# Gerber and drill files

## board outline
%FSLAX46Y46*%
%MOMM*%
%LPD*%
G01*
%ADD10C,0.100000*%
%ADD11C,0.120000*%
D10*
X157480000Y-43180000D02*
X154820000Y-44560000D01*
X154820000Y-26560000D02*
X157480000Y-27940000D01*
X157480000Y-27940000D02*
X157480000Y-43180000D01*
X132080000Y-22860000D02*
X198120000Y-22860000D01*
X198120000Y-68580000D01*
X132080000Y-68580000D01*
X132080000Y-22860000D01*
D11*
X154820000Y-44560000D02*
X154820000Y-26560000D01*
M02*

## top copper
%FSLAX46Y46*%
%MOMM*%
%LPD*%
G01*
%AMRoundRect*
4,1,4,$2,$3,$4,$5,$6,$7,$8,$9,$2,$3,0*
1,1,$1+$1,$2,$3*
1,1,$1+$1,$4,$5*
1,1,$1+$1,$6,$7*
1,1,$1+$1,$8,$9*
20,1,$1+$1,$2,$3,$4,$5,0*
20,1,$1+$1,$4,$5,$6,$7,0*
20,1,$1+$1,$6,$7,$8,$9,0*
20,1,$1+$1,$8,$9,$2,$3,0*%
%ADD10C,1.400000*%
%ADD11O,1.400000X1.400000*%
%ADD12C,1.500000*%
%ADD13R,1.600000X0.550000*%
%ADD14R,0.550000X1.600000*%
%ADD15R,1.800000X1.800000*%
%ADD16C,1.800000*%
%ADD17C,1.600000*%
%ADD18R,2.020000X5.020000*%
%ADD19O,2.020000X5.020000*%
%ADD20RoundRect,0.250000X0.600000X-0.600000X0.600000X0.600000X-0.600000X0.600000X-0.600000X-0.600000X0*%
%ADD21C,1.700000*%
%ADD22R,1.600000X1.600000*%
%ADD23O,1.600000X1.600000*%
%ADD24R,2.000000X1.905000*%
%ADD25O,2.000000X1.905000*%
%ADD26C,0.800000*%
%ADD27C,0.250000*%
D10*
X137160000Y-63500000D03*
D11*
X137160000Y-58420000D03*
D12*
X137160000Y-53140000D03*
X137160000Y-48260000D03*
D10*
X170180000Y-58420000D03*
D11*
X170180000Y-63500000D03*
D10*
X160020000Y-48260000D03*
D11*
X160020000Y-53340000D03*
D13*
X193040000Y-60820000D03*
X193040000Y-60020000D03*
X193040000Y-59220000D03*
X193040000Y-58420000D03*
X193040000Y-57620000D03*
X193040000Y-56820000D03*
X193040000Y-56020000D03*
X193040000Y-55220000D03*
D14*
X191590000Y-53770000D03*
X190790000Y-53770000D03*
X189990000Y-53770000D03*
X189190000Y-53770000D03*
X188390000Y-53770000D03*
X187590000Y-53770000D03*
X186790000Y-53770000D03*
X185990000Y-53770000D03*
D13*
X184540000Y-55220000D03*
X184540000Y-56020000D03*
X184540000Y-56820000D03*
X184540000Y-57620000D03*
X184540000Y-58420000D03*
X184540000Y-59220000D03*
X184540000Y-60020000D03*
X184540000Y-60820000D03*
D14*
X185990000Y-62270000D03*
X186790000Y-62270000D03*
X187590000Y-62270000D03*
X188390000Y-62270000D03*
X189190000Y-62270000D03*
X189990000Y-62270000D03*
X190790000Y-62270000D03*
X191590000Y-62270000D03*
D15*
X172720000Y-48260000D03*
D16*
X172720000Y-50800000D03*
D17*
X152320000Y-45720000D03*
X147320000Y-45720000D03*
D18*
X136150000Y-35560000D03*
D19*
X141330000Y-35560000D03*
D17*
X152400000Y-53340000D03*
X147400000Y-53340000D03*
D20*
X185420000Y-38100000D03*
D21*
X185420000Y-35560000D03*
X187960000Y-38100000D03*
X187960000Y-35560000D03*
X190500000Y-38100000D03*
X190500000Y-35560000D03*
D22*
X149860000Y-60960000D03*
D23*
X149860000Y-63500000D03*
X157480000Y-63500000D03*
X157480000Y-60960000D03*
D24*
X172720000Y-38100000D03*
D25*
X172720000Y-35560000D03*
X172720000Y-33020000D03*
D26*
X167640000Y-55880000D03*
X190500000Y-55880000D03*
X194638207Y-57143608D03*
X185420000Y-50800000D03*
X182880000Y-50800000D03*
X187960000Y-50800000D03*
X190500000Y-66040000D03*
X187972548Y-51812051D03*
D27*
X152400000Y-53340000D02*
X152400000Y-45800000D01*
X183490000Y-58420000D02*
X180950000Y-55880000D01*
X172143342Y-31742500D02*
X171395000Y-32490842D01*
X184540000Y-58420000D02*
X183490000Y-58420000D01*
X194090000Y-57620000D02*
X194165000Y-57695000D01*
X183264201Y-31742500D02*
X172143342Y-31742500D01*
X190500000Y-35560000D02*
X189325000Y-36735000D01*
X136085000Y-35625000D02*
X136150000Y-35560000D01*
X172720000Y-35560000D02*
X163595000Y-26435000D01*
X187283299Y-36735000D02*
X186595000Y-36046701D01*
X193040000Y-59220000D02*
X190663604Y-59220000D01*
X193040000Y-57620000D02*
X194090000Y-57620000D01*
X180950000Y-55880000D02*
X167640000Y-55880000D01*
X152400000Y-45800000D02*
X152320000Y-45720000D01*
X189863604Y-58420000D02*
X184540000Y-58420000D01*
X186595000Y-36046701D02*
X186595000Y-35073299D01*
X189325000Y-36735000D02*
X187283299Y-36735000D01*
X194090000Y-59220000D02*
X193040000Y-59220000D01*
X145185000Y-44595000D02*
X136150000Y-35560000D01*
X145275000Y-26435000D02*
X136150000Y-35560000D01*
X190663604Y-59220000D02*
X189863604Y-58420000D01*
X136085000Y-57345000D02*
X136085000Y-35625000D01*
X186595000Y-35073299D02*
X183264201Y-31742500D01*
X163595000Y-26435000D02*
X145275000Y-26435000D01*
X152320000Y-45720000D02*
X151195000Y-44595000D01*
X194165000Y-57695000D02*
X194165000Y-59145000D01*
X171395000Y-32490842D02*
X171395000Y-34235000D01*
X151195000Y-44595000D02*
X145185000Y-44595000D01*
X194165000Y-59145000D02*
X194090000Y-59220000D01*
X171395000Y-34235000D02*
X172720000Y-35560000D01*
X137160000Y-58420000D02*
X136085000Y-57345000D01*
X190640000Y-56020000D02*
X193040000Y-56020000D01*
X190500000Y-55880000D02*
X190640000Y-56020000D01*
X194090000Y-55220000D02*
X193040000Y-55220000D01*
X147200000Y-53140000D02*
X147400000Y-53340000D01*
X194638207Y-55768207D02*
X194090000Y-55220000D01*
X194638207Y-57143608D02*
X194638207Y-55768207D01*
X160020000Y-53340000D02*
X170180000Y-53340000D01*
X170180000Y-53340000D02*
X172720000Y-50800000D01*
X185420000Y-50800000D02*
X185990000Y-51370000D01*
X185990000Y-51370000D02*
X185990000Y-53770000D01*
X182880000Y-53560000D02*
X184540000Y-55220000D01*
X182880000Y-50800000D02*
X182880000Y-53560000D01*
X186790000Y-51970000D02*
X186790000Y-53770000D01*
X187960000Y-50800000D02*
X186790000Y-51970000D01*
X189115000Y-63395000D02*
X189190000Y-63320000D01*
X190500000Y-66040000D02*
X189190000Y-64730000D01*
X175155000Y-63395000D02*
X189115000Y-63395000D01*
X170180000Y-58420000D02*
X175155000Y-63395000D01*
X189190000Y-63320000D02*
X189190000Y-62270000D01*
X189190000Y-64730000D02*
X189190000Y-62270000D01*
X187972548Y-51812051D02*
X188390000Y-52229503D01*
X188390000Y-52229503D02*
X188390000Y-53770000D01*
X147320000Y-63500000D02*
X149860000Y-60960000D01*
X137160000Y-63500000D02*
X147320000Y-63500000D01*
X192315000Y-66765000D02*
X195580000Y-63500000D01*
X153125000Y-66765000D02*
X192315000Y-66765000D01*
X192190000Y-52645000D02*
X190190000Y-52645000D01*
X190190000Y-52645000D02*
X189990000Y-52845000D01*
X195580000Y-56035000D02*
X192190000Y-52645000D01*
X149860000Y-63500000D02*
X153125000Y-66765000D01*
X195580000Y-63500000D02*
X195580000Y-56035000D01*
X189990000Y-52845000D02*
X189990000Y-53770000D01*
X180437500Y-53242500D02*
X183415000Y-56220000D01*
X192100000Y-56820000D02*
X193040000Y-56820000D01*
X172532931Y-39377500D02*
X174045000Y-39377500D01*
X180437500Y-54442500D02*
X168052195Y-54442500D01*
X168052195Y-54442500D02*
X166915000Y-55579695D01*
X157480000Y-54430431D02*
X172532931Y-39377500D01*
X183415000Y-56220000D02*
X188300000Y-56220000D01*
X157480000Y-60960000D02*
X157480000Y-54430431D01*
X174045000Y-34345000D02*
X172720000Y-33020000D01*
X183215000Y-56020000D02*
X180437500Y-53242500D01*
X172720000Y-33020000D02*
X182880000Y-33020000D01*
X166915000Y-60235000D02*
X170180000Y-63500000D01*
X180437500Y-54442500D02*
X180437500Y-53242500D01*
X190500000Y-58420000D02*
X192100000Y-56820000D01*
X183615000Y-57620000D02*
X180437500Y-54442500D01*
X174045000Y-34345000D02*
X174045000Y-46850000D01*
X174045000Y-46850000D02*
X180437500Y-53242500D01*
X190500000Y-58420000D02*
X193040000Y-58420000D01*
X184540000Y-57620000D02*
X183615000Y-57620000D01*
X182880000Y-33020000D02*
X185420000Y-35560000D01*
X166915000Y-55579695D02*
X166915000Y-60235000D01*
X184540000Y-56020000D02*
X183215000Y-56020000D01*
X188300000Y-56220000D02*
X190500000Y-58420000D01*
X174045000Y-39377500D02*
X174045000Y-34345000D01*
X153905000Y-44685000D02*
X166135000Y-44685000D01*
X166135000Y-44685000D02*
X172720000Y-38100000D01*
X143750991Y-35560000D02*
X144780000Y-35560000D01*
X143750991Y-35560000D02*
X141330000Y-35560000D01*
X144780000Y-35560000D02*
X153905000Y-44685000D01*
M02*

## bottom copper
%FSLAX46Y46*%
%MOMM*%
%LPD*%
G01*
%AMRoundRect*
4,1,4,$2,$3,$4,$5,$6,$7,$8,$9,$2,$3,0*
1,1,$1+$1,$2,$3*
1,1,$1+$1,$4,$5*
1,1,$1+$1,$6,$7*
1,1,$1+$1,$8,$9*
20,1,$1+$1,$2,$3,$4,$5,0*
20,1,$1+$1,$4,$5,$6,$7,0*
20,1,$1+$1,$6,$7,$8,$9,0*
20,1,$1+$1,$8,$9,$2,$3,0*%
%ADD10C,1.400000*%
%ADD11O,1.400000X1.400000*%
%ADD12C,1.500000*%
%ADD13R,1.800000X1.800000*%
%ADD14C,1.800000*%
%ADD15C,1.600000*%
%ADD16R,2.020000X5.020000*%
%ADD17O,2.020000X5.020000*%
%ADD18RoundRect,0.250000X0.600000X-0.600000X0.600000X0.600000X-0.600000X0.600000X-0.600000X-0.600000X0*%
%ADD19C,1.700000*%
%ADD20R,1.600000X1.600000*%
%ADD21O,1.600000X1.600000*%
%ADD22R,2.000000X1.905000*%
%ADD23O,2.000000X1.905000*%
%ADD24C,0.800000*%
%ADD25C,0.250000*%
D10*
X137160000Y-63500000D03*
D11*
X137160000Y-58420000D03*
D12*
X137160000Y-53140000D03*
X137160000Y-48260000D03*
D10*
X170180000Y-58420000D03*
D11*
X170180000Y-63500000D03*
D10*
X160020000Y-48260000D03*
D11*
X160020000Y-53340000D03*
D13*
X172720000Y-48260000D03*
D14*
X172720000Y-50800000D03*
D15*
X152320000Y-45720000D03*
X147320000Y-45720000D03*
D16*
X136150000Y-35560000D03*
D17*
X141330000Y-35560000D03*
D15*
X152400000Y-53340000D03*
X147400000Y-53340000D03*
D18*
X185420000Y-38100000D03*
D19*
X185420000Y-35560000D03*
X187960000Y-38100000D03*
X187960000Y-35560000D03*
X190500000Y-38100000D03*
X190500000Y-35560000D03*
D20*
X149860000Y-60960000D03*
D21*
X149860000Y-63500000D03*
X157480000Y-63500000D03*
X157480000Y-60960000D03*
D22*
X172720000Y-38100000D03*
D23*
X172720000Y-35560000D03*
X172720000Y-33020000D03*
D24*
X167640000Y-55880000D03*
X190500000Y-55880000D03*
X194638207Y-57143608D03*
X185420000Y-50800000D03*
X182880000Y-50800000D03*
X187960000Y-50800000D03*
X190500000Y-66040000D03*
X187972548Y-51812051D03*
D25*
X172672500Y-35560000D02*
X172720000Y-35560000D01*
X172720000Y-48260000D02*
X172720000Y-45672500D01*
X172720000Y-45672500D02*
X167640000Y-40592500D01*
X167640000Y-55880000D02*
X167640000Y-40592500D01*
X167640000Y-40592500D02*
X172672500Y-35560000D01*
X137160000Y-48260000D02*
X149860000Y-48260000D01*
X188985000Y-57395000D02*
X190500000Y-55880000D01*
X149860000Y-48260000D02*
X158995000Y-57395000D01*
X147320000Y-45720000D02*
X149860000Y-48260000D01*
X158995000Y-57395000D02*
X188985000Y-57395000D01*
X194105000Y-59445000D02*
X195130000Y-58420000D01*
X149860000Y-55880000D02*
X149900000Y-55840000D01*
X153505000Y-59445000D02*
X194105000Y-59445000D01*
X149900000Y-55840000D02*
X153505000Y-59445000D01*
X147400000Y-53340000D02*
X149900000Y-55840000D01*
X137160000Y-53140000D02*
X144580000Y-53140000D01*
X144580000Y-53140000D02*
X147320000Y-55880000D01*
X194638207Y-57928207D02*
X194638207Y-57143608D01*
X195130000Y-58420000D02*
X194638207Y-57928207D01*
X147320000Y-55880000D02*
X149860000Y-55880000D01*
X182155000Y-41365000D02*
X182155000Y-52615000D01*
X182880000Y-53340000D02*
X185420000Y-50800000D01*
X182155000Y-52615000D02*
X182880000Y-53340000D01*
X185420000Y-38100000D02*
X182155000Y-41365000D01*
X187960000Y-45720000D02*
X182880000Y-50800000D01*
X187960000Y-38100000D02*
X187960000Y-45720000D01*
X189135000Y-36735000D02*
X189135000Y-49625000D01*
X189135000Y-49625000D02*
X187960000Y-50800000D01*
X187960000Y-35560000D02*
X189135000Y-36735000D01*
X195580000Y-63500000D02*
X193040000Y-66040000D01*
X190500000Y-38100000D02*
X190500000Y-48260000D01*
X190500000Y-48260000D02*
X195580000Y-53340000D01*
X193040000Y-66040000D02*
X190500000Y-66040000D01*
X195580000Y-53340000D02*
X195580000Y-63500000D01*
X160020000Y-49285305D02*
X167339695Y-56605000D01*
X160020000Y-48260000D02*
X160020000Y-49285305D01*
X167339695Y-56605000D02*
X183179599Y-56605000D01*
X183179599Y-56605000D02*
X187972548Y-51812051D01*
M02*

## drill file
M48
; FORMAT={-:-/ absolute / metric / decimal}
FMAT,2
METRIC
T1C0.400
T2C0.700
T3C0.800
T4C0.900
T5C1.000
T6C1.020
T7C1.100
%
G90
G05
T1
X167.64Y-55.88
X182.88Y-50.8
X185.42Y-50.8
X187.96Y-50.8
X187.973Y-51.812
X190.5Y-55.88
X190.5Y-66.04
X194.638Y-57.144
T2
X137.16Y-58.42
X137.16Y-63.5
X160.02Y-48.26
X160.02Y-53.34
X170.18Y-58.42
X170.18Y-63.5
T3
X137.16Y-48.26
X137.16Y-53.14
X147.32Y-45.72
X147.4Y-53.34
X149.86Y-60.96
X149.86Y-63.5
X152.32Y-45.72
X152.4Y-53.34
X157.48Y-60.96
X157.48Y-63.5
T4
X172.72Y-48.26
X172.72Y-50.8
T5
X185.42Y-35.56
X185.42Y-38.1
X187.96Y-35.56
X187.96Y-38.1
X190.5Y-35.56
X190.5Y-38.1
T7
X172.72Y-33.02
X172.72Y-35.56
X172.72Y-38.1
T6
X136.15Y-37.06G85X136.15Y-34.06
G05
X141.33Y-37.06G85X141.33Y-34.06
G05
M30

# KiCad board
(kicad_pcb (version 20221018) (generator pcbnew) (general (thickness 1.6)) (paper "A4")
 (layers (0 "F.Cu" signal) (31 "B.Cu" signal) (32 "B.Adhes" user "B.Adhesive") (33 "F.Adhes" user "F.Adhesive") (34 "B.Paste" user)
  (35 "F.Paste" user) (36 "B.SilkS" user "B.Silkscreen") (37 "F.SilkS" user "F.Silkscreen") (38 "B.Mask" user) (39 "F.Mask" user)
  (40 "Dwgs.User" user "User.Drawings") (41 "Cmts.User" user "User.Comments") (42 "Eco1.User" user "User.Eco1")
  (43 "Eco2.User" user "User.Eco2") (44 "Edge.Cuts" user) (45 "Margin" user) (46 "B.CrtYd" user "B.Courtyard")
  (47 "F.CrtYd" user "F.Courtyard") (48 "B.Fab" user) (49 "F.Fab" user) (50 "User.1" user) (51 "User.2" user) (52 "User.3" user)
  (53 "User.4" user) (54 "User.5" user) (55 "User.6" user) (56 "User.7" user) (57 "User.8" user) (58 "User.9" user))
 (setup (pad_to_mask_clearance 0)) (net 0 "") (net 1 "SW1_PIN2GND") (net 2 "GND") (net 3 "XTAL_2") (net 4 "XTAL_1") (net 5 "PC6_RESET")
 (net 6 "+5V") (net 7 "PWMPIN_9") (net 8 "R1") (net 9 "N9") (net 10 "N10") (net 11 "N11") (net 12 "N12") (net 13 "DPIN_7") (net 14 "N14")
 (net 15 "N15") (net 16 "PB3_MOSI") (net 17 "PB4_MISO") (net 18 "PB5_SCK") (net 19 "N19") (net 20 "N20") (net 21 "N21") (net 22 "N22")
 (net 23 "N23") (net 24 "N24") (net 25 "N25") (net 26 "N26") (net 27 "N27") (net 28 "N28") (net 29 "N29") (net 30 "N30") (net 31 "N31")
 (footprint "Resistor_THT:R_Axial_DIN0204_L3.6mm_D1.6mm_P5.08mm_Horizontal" (layer "F.Cu") (at 137.16 63.5 90)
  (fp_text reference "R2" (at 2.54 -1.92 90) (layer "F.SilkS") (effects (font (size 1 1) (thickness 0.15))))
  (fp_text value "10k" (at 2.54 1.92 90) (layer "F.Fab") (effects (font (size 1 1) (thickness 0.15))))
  (pad "1" thru_hole circle (at 0 0 90) (size 1.4 1.4) (drill 0.7) (layers "*.Cu" "*.Mask") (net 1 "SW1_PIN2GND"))
  (pad "2" thru_hole oval (at 5.08 0 90) (size 1.4 1.4) (drill 0.7) (layers "*.Cu" "*.Mask") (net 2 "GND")))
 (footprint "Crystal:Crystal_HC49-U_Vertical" (layer "F.Cu") (at 137.16 53.14 90)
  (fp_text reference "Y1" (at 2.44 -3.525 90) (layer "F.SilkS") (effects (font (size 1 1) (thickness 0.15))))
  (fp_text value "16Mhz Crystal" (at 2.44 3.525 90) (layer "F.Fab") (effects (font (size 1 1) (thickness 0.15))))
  (pad "1" thru_hole circle (at 0 0 90) (size 1.5 1.5) (drill 0.8) (layers "*.Cu" "*.Mask") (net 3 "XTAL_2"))
  (pad "2" thru_hole circle (at 4.88 0 90) (size 1.5 1.5) (drill 0.8) (layers "*.Cu" "*.Mask") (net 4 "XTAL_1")))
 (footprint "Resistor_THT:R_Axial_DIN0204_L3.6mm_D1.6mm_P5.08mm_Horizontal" (layer "F.Cu") (at 170.18 58.42 -90)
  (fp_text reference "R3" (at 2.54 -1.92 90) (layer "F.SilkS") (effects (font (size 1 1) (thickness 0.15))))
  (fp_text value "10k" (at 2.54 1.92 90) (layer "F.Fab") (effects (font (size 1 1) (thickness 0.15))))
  (pad "1" thru_hole circle (at 0 0 270) (size 1.4 1.4) (drill 0.7) (layers "*.Cu" "*.Mask") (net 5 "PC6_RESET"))
  (pad "2" thru_hole oval (at 5.08 0 270) (size 1.4 1.4) (drill 0.7) (layers "*.Cu" "*.Mask") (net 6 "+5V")))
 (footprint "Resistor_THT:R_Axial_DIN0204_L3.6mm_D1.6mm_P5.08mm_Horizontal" (layer "F.Cu") (at 160.02 48.26 -90)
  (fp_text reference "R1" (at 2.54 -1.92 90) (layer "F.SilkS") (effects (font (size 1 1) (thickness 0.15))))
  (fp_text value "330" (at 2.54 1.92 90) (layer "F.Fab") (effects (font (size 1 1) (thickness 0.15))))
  (pad "1" thru_hole circle (at 0 0 270) (size 1.4 1.4) (drill 0.7) (layers "*.Cu" "*.Mask") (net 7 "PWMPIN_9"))
  (pad "2" thru_hole oval (at 5.08 0 270) (size 1.4 1.4) (drill 0.7) (layers "*.Cu" "*.Mask") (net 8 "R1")))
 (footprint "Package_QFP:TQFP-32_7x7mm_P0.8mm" (layer "F.Cu") (at 188.79 58.02 180)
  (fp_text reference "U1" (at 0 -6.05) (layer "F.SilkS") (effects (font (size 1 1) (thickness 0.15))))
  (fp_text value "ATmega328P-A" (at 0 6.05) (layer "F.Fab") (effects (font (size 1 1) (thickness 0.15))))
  (pad "1" smd rect (at -4.25 -2.8 180) (size 1.6 0.55) (layers "F.Cu" "F.Paste" "F.Mask") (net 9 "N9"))
  (pad "2" smd rect (at -4.25 -2 180) (size 1.6 0.55) (layers "F.Cu" "F.Paste" "F.Mask") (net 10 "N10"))
  (pad "3" smd rect (at -4.25 -1.2 180) (size 1.6 0.55) (layers "F.Cu" "F.Paste" "F.Mask") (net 2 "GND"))
  (pad "4" smd rect (at -4.25 -0.4 180) (size 1.6 0.55) (layers "F.Cu" "F.Paste" "F.Mask") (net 6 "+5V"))
  (pad "5" smd rect (at -4.25 0.4 180) (size 1.6 0.55) (layers "F.Cu" "F.Paste" "F.Mask") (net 2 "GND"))
  (pad "6" smd rect (at -4.25 1.2 180) (size 1.6 0.55) (layers "F.Cu" "F.Paste" "F.Mask") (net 6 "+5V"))
  (pad "7" smd rect (at -4.25 2 180) (size 1.6 0.55) (layers "F.Cu" "F.Paste" "F.Mask") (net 4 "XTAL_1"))
  (pad "8" smd rect (at -4.25 2.8 180) (size 1.6 0.55) (layers "F.Cu" "F.Paste" "F.Mask") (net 3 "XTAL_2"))
  (pad "9" smd rect (at -2.8 4.25 270) (size 1.6 0.55) (layers "F.Cu" "F.Paste" "F.Mask") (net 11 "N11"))
  (pad "10" smd rect (at -2 4.25 270) (size 1.6 0.55) (layers "F.Cu" "F.Paste" "F.Mask") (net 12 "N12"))
  (pad "11" smd rect (at -1.2 4.25 270) (size 1.6 0.55) (layers "F.Cu" "F.Paste" "F.Mask") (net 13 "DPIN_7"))
  (pad "12" smd rect (at -0.4 4.25 270) (size 1.6 0.55) (layers "F.Cu" "F.Paste" "F.Mask") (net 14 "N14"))
  (pad "13" smd rect (at 0.4 4.25 270) (size 1.6 0.55) (layers "F.Cu" "F.Paste" "F.Mask") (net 7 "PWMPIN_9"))
  (pad "14" smd rect (at 1.2 4.25 270) (size 1.6 0.55) (layers "F.Cu" "F.Paste" "F.Mask") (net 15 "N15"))
  (pad "15" smd rect (at 2 4.25 270) (size 1.6 0.55) (layers "F.Cu" "F.Paste" "F.Mask") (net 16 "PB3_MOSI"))
  (pad "16" smd rect (at 2.8 4.25 270) (size 1.6 0.55) (layers "F.Cu" "F.Paste" "F.Mask") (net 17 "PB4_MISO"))
  (pad "17" smd rect (at 4.25 2.8 180) (size 1.6 0.55) (layers "F.Cu" "F.Paste" "F.Mask") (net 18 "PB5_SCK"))
  (pad "18" smd rect (at 4.25 2 180) (size 1.6 0.55) (layers "F.Cu" "F.Paste" "F.Mask") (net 6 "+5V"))
  (pad "19" smd rect (at 4.25 1.2 180) (size 1.6 0.55) (layers "F.Cu" "F.Paste" "F.Mask") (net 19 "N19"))
  (pad "20" smd rect (at 4.25 0.4 180) (size 1.6 0.55) (layers "F.Cu" "F.Paste" "F.Mask") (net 6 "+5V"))
  (pad "21" smd rect (at 4.25 -0.4 180) (size 1.6 0.55) (layers "F.Cu" "F.Paste" "F.Mask") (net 2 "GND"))
  (pad "22" smd rect (at 4.25 -1.2 180) (size 1.6 0.55) (layers "F.Cu" "F.Paste" "F.Mask") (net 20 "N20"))
  (pad "23" smd rect (at 4.25 -2 180) (size 1.6 0.55) (layers "F.Cu" "F.Paste" "F.Mask") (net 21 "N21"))
  (pad "24" smd rect (at 4.25 -2.8 180) (size 1.6 0.55) (layers "F.Cu" "F.Paste" "F.Mask") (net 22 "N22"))
  (pad "25" smd rect (at 2.8 -4.25 270) (size 1.6 0.55) (layers "F.Cu" "F.Paste" "F.Mask") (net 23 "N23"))
  (pad "26" smd rect (at 2 -4.25 270) (size 1.6 0.55) (layers "F.Cu" "F.Paste" "F.Mask") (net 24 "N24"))
  (pad "27" smd rect (at 1.2 -4.25 270) (size 1.6 0.55) (layers "F.Cu" "F.Paste" "F.Mask") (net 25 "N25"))
  (pad "28" smd rect (at 0.4 -4.25 270) (size 1.6 0.55) (layers "F.Cu" "F.Paste" "F.Mask") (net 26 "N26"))
  (pad "29" smd rect (at -0.4 -4.25 270) (size 1.6 0.55) (layers "F.Cu" "F.Paste" "F.Mask") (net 5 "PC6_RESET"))
  (pad "30" smd rect (at -1.2 -4.25 270) (size 1.6 0.55) (layers "F.Cu" "F.Paste" "F.Mask") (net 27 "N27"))
  (pad "31" smd rect (at -2 -4.25 270) (size 1.6 0.55) (layers "F.Cu" "F.Paste" "F.Mask") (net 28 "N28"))
  (pad "32" smd rect (at -2.8 -4.25 270) (size 1.6 0.55) (layers "F.Cu" "F.Paste" "F.Mask") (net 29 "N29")))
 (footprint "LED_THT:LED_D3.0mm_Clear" (layer "F.Cu") (at 172.72 48.26 -90)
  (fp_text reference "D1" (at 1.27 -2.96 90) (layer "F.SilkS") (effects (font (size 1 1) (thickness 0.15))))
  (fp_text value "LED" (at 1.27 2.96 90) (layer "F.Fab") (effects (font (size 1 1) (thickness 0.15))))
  (pad "1" thru_hole rect (at 0 0 270) (size 1.8 1.8) (drill 0.9) (layers "*.Cu" "*.Mask") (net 2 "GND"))
  (pad "2" thru_hole circle (at 2.54 0 270) (size 1.8 1.8) (drill 0.9) (layers "*.Cu" "*.Mask") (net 8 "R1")))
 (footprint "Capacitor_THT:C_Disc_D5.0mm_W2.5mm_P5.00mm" (layer "F.Cu") (at 152.32 45.72 180)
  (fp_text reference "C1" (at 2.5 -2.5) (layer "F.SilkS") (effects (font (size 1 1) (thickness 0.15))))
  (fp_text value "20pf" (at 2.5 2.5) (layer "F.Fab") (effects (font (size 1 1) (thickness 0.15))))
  (pad "1" thru_hole circle (at 0 0 180) (size 1.6 1.6) (drill 0.8) (layers "*.Cu" "*.Mask") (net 2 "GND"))
  (pad "2" thru_hole circle (at 5 0 180) (size 1.6 1.6) (drill 0.8) (layers "*.Cu" "*.Mask") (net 4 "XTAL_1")))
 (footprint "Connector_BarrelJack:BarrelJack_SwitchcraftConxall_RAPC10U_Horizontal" (layer "F.Cu") (at 136.15 35.56 180)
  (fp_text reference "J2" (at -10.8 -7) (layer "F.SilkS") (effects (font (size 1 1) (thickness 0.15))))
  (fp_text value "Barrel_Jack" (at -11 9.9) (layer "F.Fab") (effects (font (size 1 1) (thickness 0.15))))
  (fp_line (start -18.67 -9) (end -18.67 9) (stroke (width 0.12) (type solid)) (layer "Edge.Cuts"))
  (pad "1" thru_hole rect (at 0 0 180) (size 2.02 5.02) (drill oval 1.02 4.02) (layers "*.Cu" "*.Mask") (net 2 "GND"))
  (pad "2" thru_hole oval (at -5.18 0 180) (size 2.02 5.02) (drill oval 1.02 4.02) (layers "*.Cu" "*.Mask") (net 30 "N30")))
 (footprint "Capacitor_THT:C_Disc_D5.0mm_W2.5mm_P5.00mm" (layer "F.Cu") (at 152.4 53.34 180)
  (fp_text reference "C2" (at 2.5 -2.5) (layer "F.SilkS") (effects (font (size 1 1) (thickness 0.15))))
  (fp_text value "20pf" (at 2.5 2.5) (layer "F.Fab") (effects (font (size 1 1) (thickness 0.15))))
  (pad "1" thru_hole circle (at 0 0 180) (size 1.6 1.6) (drill 0.8) (layers "*.Cu" "*.Mask") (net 2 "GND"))
  (pad "2" thru_hole circle (at 5 0 180) (size 1.6 1.6) (drill 0.8) (layers "*.Cu" "*.Mask") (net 3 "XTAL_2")))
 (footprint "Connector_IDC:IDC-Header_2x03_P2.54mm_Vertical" (layer "F.Cu") (at 185.42 38.1 90)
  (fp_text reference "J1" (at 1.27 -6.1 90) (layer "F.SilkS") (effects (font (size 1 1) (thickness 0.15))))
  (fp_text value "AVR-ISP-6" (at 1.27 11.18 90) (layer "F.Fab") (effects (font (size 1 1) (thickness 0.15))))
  (pad "1" thru_hole roundrect (at 0 0 90) (size 1.7 1.7) (drill 1) (layers "*.Cu" "*.Mask") (roundrect_rratio 0.1470588235)
   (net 17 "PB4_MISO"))
  (pad "2" thru_hole circle (at 2.54 0 90) (size 1.7 1.7) (drill 1) (layers "*.Cu" "*.Mask") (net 6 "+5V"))
  (pad "3" thru_hole circle (at 0 2.54 90) (size 1.7 1.7) (drill 1) (layers "*.Cu" "*.Mask") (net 18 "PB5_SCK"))
  (pad "4" thru_hole circle (at 2.54 2.54 90) (size 1.7 1.7) (drill 1) (layers "*.Cu" "*.Mask") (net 16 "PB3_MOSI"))
  (pad "5" thru_hole circle (at 0 5.08 90) (size 1.7 1.7) (drill 1) (layers "*.Cu" "*.Mask") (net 5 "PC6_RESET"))
  (pad "6" thru_hole circle (at 2.54 5.08 90) (size 1.7 1.7) (drill 1) (layers "*.Cu" "*.Mask") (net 2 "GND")))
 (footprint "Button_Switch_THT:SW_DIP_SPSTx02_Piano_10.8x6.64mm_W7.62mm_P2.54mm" (layer "F.Cu") (at 149.86 60.96)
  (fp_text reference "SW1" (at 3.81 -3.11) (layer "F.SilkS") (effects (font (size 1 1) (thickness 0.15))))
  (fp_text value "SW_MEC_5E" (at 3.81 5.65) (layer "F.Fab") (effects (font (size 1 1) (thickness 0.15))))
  (pad "1" thru_hole rect (at 0 0) (size 1.6 1.6) (drill 0.8) (layers "*.Cu" "*.Mask") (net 1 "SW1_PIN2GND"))
  (pad "2" thru_hole oval (at 0 2.54) (size 1.6 1.6) (drill 0.8) (layers "*.Cu" "*.Mask") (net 13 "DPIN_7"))
  (pad "3" thru_hole oval (at 7.62 2.54) (size 1.6 1.6) (drill 0.8) (layers "*.Cu" "*.Mask") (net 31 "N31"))
  (pad "4" thru_hole oval (at 7.62 0) (size 1.6 1.6) (drill 0.8) (layers "*.Cu" "*.Mask") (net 6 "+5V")))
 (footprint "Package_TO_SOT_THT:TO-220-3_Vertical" (layer "F.Cu") (at 172.72 38.1 90)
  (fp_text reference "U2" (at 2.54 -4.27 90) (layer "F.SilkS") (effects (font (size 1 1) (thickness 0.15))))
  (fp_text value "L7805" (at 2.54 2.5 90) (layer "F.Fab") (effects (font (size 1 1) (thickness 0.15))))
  (pad "1" thru_hole rect (at 0 0 90) (size 1.905 2) (drill 1.1) (layers "*.Cu" "*.Mask") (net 30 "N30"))
  (pad "2" thru_hole oval (at 2.54 0 90) (size 1.905 2) (drill 1.1) (layers "*.Cu" "*.Mask") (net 2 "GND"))
  (pad "3" thru_hole oval (at 5.08 0 90) (size 1.905 2) (drill 1.1) (layers "*.Cu" "*.Mask") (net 6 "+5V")))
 (gr_line (start 157.48 43.18) (end 154.82 44.56) (stroke (width 0.1) (type default)) (layer "Edge.Cuts"))
 (gr_line (start 154.82 26.56) (end 157.48 27.94) (stroke (width 0.1) (type default)) (layer "Edge.Cuts"))
 (gr_line (start 157.48 27.94) (end 157.48 43.18) (stroke (width 0.1) (type default)) (layer "Edge.Cuts"))
 (gr_rect (start 132.08 22.86) (end 198.12 68.58) (stroke (width 0.1) (type default)) (fill none) (layer "Edge.Cuts"))
 (segment (start 152.4 53.34) (end 152.4 45.8) (width 0.25) (layer "F.Cu") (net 2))
 (segment (start 183.49 58.42) (end 180.95 55.88) (width 0.25) (layer "F.Cu") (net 2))
 (segment (start 172.143342 31.7425) (end 171.395 32.490842) (width 0.25) (layer "F.Cu") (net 2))
 (segment (start 184.54 58.42) (end 183.49 58.42) (width 0.25) (layer "F.Cu") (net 2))
 (segment (start 194.09 57.62) (end 194.165 57.695) (width 0.25) (layer "F.Cu") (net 2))
 (segment (start 183.264201 31.7425) (end 172.143342 31.7425) (width 0.25) (layer "F.Cu") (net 2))
 (segment (start 190.5 35.56) (end 189.325 36.735) (width 0.25) (layer "F.Cu") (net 2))
 (segment (start 136.085 35.625) (end 136.15 35.56) (width 0.25) (layer "F.Cu") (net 2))
 (segment (start 172.72 35.56) (end 163.595 26.435) (width 0.25) (layer "F.Cu") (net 2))
 (segment (start 187.283299 36.735) (end 186.595 36.046701) (width 0.25) (layer "F.Cu") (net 2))
 (segment (start 193.04 59.22) (end 190.663604 59.22) (width 0.25) (layer "F.Cu") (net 2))
 (segment (start 193.04 57.62) (end 194.09 57.62) (width 0.25) (layer "F.Cu") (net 2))
 (segment (start 180.95 55.88) (end 167.64 55.88) (width 0.25) (layer "F.Cu") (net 2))
 (segment (start 152.4 45.8) (end 152.32 45.72) (width 0.25) (layer "F.Cu") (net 2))
 (segment (start 189.863604 58.42) (end 184.54 58.42) (width 0.25) (layer "F.Cu") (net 2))
 (segment (start 186.595 36.046701) (end 186.595 35.073299) (width 0.25) (layer "F.Cu") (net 2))
 (segment (start 189.325 36.735) (end 187.283299 36.735) (width 0.25) (layer "F.Cu") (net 2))
 (segment (start 194.09 59.22) (end 193.04 59.22) (width 0.25) (layer "F.Cu") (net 2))
 (segment (start 145.185 44.595) (end 136.15 35.56) (width 0.25) (layer "F.Cu") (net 2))
 (segment (start 145.275 26.435) (end 136.15 35.56) (width 0.25) (layer "F.Cu") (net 2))
 (segment (start 190.663604 59.22) (end 189.863604 58.42) (width 0.25) (layer "F.Cu") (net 2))
 (segment (start 136.085 57.345) (end 136.085 35.625) (width 0.25) (layer "F.Cu") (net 2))
 (segment (start 186.595 35.073299) (end 183.264201 31.7425) (width 0.25) (layer "F.Cu") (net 2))
 (segment (start 163.595 26.435) (end 145.275 26.435) (width 0.25) (layer "F.Cu") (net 2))
 (segment (start 152.32 45.72) (end 151.195 44.595) (width 0.25) (layer "F.Cu") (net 2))
 (segment (start 194.165 57.695) (end 194.165 59.145) (width 0.25) (layer "F.Cu") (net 2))
 (segment (start 171.395 32.490842) (end 171.395 34.235) (width 0.25) (layer "F.Cu") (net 2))
 (segment (start 151.195 44.595) (end 145.185 44.595) (width 0.25) (layer "F.Cu") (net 2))
 (segment (start 194.165 59.145) (end 194.09 59.22) (width 0.25) (layer "F.Cu") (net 2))
 (segment (start 171.395 34.235) (end 172.72 35.56) (width 0.25) (layer "F.Cu") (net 2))
 (segment (start 137.16 58.42) (end 136.085 57.345) (width 0.25) (layer "F.Cu") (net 2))
 (via (at 167.64 55.88) (size 0.8) (drill 0.4) (layers "F.Cu" "B.Cu") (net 2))
 (segment (start 172.6725 35.56) (end 172.72 35.56) (width 0.25) (layer "B.Cu") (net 2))
 (segment (start 172.72 48.26) (end 172.72 45.6725) (width 0.25) (layer "B.Cu") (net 2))
 (segment (start 172.72 45.6725) (end 167.64 40.5925) (width 0.25) (layer "B.Cu") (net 2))
 (segment (start 167.64 55.88) (end 167.64 40.5925) (width 0.25) (layer "B.Cu") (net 2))
 (segment (start 167.64 40.5925) (end 172.6725 35.56) (width 0.25) (layer "B.Cu") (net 2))
 (segment (start 190.64 56.02) (end 193.04 56.02) (width 0.25) (layer "F.Cu") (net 4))
 (segment (start 190.5 55.88) (end 190.64 56.02) (width 0.25) (layer "F.Cu") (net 4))
 (via (at 190.5 55.88) (size 0.8) (drill 0.4) (layers "F.Cu" "B.Cu") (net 4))
 (segment (start 137.16 48.26) (end 149.86 48.26) (width 0.25) (layer "B.Cu") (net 4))
 (segment (start 188.985 57.395) (end 190.5 55.88) (width 0.25) (layer "B.Cu") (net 4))
 (segment (start 149.86 48.26) (end 158.995 57.395) (width 0.25) (layer "B.Cu") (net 4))
 (segment (start 147.32 45.72) (end 149.86 48.26) (width 0.25) (layer "B.Cu") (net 4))
 (segment (start 158.995 57.395) (end 188.985 57.395) (width 0.25) (layer "B.Cu") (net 4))
 (segment (start 194.09 55.22) (end 193.04 55.22) (width 0.25) (layer "F.Cu") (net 3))
 (segment (start 147.2 53.14) (end 147.4 53.34) (width 0.25) (layer "F.Cu") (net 3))
 (segment (start 194.638207 55.768207) (end 194.09 55.22) (width 0.25) (layer "F.Cu") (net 3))
 (segment (start 194.638207 57.143608) (end 194.638207 55.768207) (width 0.25) (layer "F.Cu") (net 3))
 (via (at 194.638207 57.143608) (size 0.8) (drill 0.4) (layers "F.Cu" "B.Cu") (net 3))
 (segment (start 194.105 59.445) (end 195.13 58.42) (width 0.25) (layer "B.Cu") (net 3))
 (segment (start 149.86 55.88) (end 149.9 55.84) (width 0.25) (layer "B.Cu") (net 3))
 (segment (start 153.505 59.445) (end 194.105 59.445) (width 0.25) (layer "B.Cu") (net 3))
 (segment (start 149.9 55.84) (end 153.505 59.445) (width 0.25) (layer "B.Cu") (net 3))
 (segment (start 147.4 53.34) (end 149.9 55.84) (width 0.25) (layer "B.Cu") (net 3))
 (segment (start 137.16 53.14) (end 144.58 53.14) (width 0.25) (layer "B.Cu") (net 3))
 (segment (start 144.58 53.14) (end 147.32 55.88) (width 0.25) (layer "B.Cu") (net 3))
 (segment (start 194.638207 57.928207) (end 194.638207 57.143608) (width 0.25) (layer "B.Cu") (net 3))
 (segment (start 195.13 58.42) (end 194.638207 57.928207) (width 0.25) (layer "B.Cu") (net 3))
 (segment (start 147.32 55.88) (end 149.86 55.88) (width 0.25) (layer "B.Cu") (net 3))
 (segment (start 160.02 53.34) (end 170.18 53.34) (width 0.25) (layer "F.Cu") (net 8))
 (segment (start 170.18 53.34) (end 172.72 50.8) (width 0.25) (layer "F.Cu") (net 8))
 (segment (start 185.42 50.8) (end 185.99 51.37) (width 0.25) (layer "F.Cu") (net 17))
 (segment (start 185.99 51.37) (end 185.99 53.77) (width 0.25) (layer "F.Cu") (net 17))
 (via (at 185.42 50.8) (size 0.8) (drill 0.4) (layers "F.Cu" "B.Cu") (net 17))
 (segment (start 182.155 41.365) (end 182.155 52.615) (width 0.25) (layer "B.Cu") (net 17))
 (segment (start 182.88 53.34) (end 185.42 50.8) (width 0.25) (layer "B.Cu") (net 17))
 (segment (start 182.155 52.615) (end 182.88 53.34) (width 0.25) (layer "B.Cu") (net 17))
 (segment (start 185.42 38.1) (end 182.155 41.365) (width 0.25) (layer "B.Cu") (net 17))
 (segment (start 182.88 53.56) (end 184.54 55.22) (width 0.25) (layer "F.Cu") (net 18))
 (segment (start 182.88 50.8) (end 182.88 53.56) (width 0.25) (layer "F.Cu") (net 18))
 (via (at 182.88 50.8) (size 0.8) (drill 0.4) (layers "F.Cu" "B.Cu") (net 18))
 (segment (start 187.96 45.72) (end 182.88 50.8) (width 0.25) (layer "B.Cu") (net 18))
 (segment (start 187.96 38.1) (end 187.96 45.72) (width 0.25) (layer "B.Cu") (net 18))
 (segment (start 186.79 51.97) (end 186.79 53.77) (width 0.25) (layer "F.Cu") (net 16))
 (segment (start 187.96 50.8) (end 186.79 51.97) (width 0.25) (layer "F.Cu") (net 16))
 (via (at 187.96 50.8) (size 0.8) (drill 0.4) (layers "F.Cu" "B.Cu") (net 16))
 (segment (start 189.135 36.735) (end 189.135 49.625) (width 0.25) (layer "B.Cu") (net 16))
 (segment (start 189.135 49.625) (end 187.96 50.8) (width 0.25) (layer "B.Cu") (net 16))
 (segment (start 187.96 35.56) (end 189.135 36.735) (width 0.25) (layer "B.Cu") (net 16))
 (segment (start 189.115 63.395) (end 189.19 63.32) (width 0.25) (layer "F.Cu") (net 5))
 (segment (start 190.5 66.04) (end 189.19 64.73) (width 0.25) (layer "F.Cu") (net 5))
 (segment (start 175.155 63.395) (end 189.115 63.395) (width 0.25) (layer "F.Cu") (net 5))
 (segment (start 170.18 58.42) (end 175.155 63.395) (width 0.25) (layer "F.Cu") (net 5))
 (segment (start 189.19 63.32) (end 189.19 62.27) (width 0.25) (layer "F.Cu") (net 5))
 (segment (start 189.19 64.73) (end 189.19 62.27) (width 0.25) (layer "F.Cu") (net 5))
 (via (at 190.5 66.04) (size 0.8) (drill 0.4) (layers "F.Cu" "B.Cu") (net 5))
 (segment (start 195.58 63.5) (end 193.04 66.04) (width 0.25) (layer "B.Cu") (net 5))
 (segment (start 190.5 38.1) (end 190.5 48.26) (width 0.25) (layer "B.Cu") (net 5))
 (segment (start 190.5 48.26) (end 195.58 53.34) (width 0.25) (layer "B.Cu") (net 5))
 (segment (start 193.04 66.04) (end 190.5 66.04) (width 0.25) (layer "B.Cu") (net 5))
 (segment (start 195.58 53.34) (end 195.58 63.5) (width 0.25) (layer "B.Cu") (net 5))
 (segment (start 187.972548 51.812051) (end 188.39 52.229503) (width 0.25) (layer "F.Cu") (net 7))
 (segment (start 188.39 52.229503) (end 188.39 53.77) (width 0.25) (layer "F.Cu") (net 7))
 (via (at 187.972548 51.812051) (size 0.8) (drill 0.4) (layers "F.Cu" "B.Cu") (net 7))
 (segment (start 160.02 49.285305) (end 167.339695 56.605) (width 0.25) (layer "B.Cu") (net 7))
 (segment (start 160.02 48.26) (end 160.02 49.285305) (width 0.25) (layer "B.Cu") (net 7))
 (segment (start 167.339695 56.605) (end 183.179599 56.605) (width 0.25) (layer "B.Cu") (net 7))
 (segment (start 183.179599 56.605) (end 187.972548 51.812051) (width 0.25) (layer "B.Cu") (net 7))
 (segment (start 147.32 63.5) (end 149.86 60.96) (width 0.25) (layer "F.Cu") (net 1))
 (segment (start 137.16 63.5) (end 147.32 63.5) (width 0.25) (layer "F.Cu") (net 1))
 (segment (start 192.315 66.765) (end 195.58 63.5) (width 0.25) (layer "F.Cu") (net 13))
 (segment (start 153.125 66.765) (end 192.315 66.765) (width 0.25) (layer "F.Cu") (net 13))
 (segment (start 192.19 52.645) (end 190.19 52.645) (width 0.25) (layer "F.Cu") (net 13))
 (segment (start 190.19 52.645) (end 189.99 52.845) (width 0.25) (layer "F.Cu") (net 13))
 (segment (start 195.58 56.035) (end 192.19 52.645) (width 0.25) (layer "F.Cu") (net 13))
 (segment (start 149.86 63.5) (end 153.125 66.765) (width 0.25) (layer "F.Cu") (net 13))
 (segment (start 195.58 63.5) (end 195.58 56.035) (width 0.25) (layer "F.Cu") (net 13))
 (segment (start 189.99 52.845) (end 189.99 53.77) (width 0.25) (layer "F.Cu") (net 13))
 (segment (start 180.4375 53.2425) (end 183.415 56.22) (width 0.25) (layer "F.Cu") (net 6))
 (segment (start 192.1 56.82) (end 193.04 56.82) (width 0.25) (layer "F.Cu") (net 6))
 (segment (start 172.532931 39.3775) (end 174.045 39.3775) (width 0.25) (layer "F.Cu") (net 6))
 (segment (start 180.4375 54.4425) (end 168.052195 54.4425) (width 0.25) (layer "F.Cu") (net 6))
 (segment (start 168.052195 54.4425) (end 166.915 55.579695) (width 0.25) (layer "F.Cu") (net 6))
 (segment (start 157.48 54.430431) (end 172.532931 39.3775) (width 0.25) (layer "F.Cu") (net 6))
 (segment (start 183.415 56.22) (end 188.3 56.22) (width 0.25) (layer "F.Cu") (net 6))
 (segment (start 157.48 60.96) (end 157.48 54.430431) (width 0.25) (layer "F.Cu") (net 6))
 (segment (start 174.045 34.345) (end 172.72 33.02) (width 0.25) (layer "F.Cu") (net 6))
 (segment (start 183.215 56.02) (end 180.4375 53.2425) (width 0.25) (layer "F.Cu") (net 6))
 (segment (start 172.72 33.02) (end 182.88 33.02) (width 0.25) (layer "F.Cu") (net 6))
 (segment (start 166.915 60.235) (end 170.18 63.5) (width 0.25) (layer "F.Cu") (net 6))
 (segment (start 180.4375 54.4425) (end 180.4375 53.2425) (width 0.25) (layer "F.Cu") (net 6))
 (segment (start 190.5 58.42) (end 192.1 56.82) (width 0.25) (layer "F.Cu") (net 6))
 (segment (start 183.615 57.62) (end 180.4375 54.4425) (width 0.25) (layer "F.Cu") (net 6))
 (segment (start 174.045 34.345) (end 174.045 46.85) (width 0.25) (layer "F.Cu") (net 6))
 (segment (start 174.045 46.85) (end 180.4375 53.2425) (width 0.25) (layer "F.Cu") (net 6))
 (segment (start 190.5 58.42) (end 193.04 58.42) (width 0.25) (layer "F.Cu") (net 6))
 (segment (start 184.54 57.62) (end 183.615 57.62) (width 0.25) (layer "F.Cu") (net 6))
 (segment (start 182.88 33.02) (end 185.42 35.56) (width 0.25) (layer "F.Cu") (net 6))
 (segment (start 166.915 55.579695) (end 166.915 60.235) (width 0.25) (layer "F.Cu") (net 6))
 (segment (start 184.54 56.02) (end 183.215 56.02) (width 0.25) (layer "F.Cu") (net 6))
 (segment (start 188.3 56.22) (end 190.5 58.42) (width 0.25) (layer "F.Cu") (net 6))
 (segment (start 174.045 39.3775) (end 174.045 34.345) (width 0.25) (layer "F.Cu") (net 6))
 (segment (start 153.905 44.685) (end 166.135 44.685) (width 0.25) (layer "F.Cu") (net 30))
 (segment (start 166.135 44.685) (end 172.72 38.1) (width 0.25) (layer "F.Cu") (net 30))
 (segment (start 143.750991 35.56) (end 144.78 35.56) (width 0.25) (layer "F.Cu") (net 30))
 (segment (start 143.750991 35.56) (end 141.33 35.56) (width 0.25) (layer "F.Cu") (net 30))
 (segment (start 144.78 35.56) (end 153.905 44.685) (width 0.25) (layer "F.Cu") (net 30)))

